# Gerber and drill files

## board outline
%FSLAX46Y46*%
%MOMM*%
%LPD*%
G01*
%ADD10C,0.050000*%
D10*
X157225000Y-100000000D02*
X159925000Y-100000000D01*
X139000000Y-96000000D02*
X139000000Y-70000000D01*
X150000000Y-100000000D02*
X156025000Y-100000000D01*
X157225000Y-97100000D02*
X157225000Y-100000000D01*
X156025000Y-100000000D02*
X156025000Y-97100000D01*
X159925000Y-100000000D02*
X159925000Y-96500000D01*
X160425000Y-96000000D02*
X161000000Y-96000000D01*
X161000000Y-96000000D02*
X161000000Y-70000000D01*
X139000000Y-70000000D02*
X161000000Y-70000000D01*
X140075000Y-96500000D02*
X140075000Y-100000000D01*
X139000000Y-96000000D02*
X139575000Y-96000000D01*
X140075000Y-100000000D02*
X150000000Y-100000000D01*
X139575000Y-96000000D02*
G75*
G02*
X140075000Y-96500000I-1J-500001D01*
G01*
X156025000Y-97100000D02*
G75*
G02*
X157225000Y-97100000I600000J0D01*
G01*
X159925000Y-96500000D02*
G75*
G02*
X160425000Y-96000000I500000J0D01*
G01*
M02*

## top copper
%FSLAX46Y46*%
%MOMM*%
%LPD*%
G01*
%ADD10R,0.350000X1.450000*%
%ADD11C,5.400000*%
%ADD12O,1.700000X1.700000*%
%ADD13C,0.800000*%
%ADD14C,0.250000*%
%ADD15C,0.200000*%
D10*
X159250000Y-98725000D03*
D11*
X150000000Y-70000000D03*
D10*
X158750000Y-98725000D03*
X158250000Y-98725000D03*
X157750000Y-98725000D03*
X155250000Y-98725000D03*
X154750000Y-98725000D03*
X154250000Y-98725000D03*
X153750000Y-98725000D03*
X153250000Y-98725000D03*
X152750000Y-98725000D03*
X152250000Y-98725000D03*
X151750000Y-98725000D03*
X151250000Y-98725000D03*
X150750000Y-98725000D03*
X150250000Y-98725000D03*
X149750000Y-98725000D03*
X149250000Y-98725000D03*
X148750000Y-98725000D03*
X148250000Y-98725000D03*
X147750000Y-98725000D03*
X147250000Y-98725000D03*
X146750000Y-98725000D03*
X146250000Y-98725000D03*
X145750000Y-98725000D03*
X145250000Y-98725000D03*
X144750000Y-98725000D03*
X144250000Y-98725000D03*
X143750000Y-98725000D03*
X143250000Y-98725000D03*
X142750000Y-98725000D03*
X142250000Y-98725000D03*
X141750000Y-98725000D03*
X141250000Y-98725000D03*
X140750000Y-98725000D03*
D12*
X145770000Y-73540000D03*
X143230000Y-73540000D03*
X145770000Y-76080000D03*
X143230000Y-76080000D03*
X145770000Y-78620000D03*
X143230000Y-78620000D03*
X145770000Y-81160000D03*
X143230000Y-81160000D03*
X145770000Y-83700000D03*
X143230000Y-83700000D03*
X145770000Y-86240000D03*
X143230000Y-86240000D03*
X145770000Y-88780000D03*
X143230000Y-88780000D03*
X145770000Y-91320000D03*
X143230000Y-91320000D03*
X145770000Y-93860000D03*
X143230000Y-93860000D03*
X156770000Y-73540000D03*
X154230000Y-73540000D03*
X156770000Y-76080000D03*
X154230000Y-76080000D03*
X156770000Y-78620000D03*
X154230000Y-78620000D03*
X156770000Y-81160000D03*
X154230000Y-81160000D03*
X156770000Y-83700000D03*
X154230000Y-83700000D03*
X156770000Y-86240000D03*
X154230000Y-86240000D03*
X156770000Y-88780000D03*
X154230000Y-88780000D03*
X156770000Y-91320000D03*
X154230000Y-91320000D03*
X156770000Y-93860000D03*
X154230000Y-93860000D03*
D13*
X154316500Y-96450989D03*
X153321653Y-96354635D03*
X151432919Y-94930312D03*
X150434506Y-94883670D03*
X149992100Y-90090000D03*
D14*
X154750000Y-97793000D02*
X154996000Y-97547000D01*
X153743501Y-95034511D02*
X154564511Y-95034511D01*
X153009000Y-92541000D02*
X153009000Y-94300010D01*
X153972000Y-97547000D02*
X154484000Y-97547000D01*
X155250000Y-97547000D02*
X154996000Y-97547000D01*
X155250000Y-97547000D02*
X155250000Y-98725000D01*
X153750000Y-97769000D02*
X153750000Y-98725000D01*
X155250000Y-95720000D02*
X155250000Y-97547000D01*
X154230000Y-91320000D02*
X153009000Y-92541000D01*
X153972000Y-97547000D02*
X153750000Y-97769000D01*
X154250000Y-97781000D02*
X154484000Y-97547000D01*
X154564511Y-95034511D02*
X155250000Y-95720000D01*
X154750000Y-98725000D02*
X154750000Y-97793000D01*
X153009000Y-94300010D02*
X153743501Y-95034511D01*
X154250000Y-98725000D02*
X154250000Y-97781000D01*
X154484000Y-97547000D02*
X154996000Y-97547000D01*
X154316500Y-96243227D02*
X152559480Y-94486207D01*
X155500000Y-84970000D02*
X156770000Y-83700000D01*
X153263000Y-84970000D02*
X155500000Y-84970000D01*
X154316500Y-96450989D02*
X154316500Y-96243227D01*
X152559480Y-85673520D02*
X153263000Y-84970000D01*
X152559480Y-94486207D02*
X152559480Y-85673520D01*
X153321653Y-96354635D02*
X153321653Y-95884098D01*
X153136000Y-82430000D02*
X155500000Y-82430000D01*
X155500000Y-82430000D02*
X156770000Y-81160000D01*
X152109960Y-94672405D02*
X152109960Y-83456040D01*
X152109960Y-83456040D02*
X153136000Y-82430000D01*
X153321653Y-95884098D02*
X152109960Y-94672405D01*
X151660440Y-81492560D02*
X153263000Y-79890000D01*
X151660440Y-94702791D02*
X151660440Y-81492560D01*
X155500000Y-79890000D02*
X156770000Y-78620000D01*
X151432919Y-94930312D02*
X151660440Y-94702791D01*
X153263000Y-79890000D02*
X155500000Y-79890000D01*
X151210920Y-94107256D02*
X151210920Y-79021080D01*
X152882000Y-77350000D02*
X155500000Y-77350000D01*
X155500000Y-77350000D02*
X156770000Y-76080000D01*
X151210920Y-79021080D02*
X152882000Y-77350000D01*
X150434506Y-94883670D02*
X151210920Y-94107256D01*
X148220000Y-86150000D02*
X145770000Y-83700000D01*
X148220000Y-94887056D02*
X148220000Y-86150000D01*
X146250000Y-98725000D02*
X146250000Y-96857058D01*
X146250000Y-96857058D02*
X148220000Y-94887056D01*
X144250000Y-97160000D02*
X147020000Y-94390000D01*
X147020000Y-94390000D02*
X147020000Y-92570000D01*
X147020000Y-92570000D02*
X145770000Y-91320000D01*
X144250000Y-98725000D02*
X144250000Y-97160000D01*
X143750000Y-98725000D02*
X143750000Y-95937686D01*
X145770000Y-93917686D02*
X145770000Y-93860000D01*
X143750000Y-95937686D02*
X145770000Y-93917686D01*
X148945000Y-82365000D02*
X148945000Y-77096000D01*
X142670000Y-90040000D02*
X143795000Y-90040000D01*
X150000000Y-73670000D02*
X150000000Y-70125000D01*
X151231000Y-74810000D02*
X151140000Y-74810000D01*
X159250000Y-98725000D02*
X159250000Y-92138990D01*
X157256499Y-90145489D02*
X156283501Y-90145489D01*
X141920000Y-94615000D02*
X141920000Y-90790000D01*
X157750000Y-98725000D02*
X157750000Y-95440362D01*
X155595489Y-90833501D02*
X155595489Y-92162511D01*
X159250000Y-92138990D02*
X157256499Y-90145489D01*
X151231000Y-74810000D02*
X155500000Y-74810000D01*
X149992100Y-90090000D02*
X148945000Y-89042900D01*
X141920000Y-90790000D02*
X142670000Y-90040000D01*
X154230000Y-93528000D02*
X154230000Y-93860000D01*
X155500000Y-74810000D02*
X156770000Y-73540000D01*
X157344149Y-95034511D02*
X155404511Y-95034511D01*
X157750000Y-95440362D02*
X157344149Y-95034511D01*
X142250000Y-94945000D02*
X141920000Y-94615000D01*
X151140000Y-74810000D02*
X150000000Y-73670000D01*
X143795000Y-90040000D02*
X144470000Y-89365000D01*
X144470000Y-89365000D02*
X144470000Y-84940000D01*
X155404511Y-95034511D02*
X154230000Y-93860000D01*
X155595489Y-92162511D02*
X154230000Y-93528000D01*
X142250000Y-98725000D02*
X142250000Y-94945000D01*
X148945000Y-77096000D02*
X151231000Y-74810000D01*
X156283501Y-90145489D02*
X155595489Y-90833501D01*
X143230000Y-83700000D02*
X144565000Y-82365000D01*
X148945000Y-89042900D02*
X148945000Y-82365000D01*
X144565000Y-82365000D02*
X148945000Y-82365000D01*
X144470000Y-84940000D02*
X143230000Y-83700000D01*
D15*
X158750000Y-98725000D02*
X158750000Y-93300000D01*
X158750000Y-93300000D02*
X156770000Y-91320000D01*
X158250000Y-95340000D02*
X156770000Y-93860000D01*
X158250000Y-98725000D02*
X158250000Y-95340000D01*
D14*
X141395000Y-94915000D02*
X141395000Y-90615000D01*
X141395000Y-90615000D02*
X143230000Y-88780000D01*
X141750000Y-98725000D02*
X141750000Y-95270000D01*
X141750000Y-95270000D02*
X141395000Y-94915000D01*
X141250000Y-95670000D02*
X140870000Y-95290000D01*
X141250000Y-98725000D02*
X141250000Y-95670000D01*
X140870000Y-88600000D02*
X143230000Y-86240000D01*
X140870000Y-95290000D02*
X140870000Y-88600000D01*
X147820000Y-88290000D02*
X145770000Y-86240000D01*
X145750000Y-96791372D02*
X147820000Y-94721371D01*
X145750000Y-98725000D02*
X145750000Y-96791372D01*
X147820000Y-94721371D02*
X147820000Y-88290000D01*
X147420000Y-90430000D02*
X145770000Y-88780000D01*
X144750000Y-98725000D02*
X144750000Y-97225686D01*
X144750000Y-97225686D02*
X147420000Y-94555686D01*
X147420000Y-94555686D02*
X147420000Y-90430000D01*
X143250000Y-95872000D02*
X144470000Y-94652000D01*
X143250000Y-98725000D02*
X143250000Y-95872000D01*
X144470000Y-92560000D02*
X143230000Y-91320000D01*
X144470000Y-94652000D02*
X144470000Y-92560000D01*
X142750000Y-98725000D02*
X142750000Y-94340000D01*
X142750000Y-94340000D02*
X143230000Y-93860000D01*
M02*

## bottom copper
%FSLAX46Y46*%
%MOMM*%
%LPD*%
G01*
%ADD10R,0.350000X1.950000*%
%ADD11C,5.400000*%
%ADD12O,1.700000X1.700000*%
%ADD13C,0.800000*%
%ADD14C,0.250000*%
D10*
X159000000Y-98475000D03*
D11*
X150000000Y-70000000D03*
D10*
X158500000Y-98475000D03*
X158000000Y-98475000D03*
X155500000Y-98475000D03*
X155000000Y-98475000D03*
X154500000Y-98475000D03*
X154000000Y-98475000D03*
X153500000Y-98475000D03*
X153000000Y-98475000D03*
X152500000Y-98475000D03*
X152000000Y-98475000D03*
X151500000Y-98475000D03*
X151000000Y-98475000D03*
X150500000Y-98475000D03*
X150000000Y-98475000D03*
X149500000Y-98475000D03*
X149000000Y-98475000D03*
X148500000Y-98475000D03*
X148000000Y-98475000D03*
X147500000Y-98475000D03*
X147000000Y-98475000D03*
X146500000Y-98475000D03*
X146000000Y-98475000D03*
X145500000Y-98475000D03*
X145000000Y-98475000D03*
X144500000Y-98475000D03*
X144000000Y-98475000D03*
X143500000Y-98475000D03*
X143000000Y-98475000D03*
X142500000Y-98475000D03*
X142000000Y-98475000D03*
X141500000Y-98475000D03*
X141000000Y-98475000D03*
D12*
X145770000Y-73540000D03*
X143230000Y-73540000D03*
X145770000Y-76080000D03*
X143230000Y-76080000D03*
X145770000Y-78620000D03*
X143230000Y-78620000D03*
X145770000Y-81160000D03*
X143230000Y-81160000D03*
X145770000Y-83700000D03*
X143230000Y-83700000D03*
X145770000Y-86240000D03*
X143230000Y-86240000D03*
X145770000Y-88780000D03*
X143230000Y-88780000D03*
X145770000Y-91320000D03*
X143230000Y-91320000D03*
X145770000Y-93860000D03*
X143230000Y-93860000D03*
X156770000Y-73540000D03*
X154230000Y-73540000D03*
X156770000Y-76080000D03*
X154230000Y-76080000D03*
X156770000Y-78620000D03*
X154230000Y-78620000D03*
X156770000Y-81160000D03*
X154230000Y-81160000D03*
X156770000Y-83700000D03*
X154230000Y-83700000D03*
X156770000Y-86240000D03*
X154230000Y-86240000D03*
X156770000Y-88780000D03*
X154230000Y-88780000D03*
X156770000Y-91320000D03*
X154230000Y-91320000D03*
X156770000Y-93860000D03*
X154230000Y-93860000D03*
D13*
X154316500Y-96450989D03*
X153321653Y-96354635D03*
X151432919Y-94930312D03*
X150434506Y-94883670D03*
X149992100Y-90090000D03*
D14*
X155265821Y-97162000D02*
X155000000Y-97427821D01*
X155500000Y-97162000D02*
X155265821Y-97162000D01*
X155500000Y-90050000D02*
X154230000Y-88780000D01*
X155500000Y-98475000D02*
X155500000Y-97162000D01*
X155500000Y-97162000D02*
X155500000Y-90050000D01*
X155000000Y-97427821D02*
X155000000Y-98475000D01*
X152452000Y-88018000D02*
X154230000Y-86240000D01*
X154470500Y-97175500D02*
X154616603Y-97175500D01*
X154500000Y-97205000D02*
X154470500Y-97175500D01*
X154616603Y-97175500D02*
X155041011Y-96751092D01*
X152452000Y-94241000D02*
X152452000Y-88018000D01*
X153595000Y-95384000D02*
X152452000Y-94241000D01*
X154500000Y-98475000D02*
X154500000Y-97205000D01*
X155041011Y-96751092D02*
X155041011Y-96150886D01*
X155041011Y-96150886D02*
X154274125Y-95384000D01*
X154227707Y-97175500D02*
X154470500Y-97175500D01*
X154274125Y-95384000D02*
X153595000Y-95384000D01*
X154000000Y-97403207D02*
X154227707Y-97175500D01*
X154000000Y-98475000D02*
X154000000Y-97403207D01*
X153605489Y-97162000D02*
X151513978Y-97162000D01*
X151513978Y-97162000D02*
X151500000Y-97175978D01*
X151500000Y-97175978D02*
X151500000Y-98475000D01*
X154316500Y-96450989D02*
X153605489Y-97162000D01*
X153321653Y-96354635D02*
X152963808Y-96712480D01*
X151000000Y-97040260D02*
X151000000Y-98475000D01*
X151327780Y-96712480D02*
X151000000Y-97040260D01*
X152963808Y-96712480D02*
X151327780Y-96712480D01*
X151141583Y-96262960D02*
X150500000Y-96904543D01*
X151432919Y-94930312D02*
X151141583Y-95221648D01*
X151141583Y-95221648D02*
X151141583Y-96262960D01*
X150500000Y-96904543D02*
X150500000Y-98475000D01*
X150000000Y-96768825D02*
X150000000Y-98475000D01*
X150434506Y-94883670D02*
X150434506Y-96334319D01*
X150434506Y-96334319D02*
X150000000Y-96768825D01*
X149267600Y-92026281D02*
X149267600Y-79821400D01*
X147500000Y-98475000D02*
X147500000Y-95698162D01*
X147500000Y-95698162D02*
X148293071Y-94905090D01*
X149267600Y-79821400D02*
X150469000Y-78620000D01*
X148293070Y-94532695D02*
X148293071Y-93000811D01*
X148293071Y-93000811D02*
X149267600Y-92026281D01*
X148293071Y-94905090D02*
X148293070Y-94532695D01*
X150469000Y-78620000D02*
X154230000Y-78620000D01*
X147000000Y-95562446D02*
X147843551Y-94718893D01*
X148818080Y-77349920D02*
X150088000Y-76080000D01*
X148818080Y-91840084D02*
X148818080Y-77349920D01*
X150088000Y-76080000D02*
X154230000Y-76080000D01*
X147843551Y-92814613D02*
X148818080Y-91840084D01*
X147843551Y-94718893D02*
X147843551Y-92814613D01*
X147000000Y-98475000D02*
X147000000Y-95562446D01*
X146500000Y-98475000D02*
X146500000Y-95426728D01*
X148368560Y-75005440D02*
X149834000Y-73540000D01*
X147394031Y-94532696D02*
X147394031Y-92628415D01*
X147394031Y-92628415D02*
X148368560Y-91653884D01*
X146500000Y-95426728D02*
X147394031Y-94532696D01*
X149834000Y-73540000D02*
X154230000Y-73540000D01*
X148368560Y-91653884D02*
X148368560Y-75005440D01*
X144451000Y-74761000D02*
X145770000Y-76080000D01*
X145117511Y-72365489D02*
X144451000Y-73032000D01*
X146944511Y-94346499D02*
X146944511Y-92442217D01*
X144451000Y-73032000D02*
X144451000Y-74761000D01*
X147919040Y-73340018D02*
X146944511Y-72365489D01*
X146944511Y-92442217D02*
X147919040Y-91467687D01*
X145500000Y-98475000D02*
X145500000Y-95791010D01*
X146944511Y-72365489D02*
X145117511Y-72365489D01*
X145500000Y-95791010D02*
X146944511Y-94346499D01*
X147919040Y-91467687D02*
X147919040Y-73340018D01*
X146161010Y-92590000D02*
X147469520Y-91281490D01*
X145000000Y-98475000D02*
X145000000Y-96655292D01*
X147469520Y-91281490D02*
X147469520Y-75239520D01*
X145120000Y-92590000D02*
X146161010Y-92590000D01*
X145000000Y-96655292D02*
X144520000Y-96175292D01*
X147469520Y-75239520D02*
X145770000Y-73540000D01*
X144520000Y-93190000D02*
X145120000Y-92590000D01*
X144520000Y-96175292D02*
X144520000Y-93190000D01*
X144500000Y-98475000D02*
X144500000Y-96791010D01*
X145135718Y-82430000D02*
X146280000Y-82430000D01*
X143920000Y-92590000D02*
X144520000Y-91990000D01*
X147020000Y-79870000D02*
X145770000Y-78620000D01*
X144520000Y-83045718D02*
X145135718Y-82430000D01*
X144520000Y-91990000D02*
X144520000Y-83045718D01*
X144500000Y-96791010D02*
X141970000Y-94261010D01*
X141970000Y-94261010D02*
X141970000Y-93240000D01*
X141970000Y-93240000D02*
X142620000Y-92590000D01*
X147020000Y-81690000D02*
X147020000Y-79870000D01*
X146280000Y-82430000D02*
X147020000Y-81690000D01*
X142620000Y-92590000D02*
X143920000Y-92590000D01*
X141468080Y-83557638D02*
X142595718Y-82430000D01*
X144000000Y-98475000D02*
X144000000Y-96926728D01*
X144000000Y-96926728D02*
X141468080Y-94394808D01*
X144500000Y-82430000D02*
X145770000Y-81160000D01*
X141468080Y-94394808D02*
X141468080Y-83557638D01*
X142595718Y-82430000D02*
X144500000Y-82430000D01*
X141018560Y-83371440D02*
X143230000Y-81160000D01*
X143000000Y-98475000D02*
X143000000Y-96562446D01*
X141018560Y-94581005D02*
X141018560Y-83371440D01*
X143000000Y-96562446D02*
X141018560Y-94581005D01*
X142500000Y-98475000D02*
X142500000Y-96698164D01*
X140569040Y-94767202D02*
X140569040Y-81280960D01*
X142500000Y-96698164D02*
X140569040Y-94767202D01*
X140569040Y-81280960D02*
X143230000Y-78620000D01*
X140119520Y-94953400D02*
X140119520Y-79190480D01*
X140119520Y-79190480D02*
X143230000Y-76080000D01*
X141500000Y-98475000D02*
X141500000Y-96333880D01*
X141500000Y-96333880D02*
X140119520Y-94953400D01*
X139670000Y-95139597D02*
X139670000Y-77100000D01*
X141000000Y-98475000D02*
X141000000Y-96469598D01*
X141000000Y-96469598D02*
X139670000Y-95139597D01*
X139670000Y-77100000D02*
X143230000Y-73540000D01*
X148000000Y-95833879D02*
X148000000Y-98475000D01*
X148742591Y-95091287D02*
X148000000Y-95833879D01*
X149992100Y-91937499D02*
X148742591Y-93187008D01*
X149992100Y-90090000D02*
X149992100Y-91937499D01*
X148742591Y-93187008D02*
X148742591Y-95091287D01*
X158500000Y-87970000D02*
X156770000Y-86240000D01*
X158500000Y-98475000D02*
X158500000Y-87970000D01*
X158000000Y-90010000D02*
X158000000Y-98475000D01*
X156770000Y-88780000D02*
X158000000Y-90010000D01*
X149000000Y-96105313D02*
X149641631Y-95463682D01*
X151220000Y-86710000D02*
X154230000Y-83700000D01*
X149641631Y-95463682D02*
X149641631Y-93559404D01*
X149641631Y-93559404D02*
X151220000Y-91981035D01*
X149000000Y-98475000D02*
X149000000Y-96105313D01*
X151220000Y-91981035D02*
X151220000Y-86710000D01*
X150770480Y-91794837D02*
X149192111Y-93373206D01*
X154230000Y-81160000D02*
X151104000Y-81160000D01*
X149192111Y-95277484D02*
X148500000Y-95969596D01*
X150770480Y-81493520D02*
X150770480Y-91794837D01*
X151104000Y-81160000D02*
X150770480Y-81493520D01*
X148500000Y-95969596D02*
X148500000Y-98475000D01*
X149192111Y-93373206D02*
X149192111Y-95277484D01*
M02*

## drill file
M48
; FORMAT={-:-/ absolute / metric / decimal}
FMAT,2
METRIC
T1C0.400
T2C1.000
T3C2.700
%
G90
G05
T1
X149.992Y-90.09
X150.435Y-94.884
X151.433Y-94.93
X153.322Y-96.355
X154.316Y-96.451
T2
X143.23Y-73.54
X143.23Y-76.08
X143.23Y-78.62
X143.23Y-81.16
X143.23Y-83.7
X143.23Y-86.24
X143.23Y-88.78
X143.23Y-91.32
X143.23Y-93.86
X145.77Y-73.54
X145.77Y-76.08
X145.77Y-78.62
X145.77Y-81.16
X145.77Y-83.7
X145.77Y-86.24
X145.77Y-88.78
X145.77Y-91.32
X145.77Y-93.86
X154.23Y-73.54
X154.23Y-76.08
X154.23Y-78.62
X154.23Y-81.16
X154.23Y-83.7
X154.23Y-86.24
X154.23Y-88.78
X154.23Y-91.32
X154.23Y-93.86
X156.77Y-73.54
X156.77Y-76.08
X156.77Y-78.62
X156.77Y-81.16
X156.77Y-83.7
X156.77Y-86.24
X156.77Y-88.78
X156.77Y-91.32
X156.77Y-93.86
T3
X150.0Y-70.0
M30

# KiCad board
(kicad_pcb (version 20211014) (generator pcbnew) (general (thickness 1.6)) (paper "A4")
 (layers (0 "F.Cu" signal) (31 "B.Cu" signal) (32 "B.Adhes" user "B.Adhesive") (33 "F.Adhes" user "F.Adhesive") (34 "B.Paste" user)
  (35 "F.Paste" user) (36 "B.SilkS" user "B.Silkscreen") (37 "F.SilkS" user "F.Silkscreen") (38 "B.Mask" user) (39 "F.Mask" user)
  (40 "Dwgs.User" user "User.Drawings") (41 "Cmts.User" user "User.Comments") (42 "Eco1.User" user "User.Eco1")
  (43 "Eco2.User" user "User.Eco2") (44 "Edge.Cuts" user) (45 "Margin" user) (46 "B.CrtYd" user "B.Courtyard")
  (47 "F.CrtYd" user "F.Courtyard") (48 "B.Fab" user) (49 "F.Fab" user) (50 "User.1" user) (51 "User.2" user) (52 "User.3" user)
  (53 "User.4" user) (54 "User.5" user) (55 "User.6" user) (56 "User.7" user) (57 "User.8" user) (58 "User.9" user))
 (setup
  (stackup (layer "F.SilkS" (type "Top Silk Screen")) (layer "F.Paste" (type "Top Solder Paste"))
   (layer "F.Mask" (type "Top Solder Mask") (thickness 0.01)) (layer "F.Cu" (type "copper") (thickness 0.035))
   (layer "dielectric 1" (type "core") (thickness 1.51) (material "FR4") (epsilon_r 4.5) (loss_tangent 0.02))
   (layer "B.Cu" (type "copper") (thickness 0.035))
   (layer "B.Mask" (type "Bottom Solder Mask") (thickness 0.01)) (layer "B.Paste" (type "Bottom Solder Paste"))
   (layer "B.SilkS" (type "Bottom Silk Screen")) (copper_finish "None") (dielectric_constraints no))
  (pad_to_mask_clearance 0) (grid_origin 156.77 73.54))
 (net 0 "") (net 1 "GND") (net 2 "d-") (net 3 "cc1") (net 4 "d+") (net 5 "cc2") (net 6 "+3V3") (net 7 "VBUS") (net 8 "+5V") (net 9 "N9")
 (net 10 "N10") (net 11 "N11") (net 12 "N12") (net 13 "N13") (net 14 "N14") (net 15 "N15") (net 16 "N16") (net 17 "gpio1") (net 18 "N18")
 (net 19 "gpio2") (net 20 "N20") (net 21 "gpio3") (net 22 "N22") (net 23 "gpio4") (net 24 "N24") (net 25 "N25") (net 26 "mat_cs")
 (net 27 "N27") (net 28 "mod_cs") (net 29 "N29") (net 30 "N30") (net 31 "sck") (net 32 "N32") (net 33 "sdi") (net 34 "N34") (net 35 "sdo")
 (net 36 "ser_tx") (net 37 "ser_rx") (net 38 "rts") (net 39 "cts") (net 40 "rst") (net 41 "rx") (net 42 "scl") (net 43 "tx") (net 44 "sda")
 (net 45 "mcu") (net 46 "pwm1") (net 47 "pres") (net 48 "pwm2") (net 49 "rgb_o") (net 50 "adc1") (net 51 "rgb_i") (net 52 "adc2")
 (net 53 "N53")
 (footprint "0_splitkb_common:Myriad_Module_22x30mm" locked (layer "F.Cu") (at 150 100)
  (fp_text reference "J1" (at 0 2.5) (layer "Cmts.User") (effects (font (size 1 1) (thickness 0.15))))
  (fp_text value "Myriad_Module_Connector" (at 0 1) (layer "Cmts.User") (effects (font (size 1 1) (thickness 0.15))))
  (fp_line (start 7.225 0) (end 9.925 0) (layer "Edge.Cuts") (width 0.05))
  (fp_line (start -11 -4) (end -11 -30) (layer "Edge.Cuts") (width 0.05))
  (fp_line (start 0 0) (end 6.025 0) (layer "Edge.Cuts") (width 0.05))
  (fp_line (start 7.225 -2.9) (end 7.225 0) (layer "Edge.Cuts") (width 0.05))
  (fp_line (start 6.025 0) (end 6.025 -2.9) (layer "Edge.Cuts") (width 0.05))
  (fp_line (start 9.925 0) (end 9.925 -3.5) (layer "Edge.Cuts") (width 0.05))
  (fp_line (start 10.425 -4) (end 11 -4) (layer "Edge.Cuts") (width 0.05))
  (fp_line (start 11 -4) (end 11 -30) (layer "Edge.Cuts") (width 0.05))
  (fp_line (start -11 -30) (end 11 -30) (layer "Edge.Cuts") (width 0.05))
  (fp_line (start -9.925 -3.5) (end -9.925 0) (layer "Edge.Cuts") (width 0.05))
  (fp_line (start -11 -4) (end -10.425 -4) (layer "Edge.Cuts") (width 0.05))
  (fp_line (start -9.925 0) (end 0 0) (layer "Edge.Cuts") (width 0.05))
  (fp_arc (start -10.425 -4) (mid -10.071447 -3.853553) (end -9.925 -3.5) (layer "Edge.Cuts") (width 0.05))
  (fp_arc (start 6.025 -2.9) (mid 6.625 -3.5) (end 7.225 -2.9) (layer "Edge.Cuts") (width 0.05))
  (fp_arc (start 9.925 -3.5) (mid 10.071447 -3.853553) (end 10.425 -4) (layer "Edge.Cuts") (width 0.05))
  (pad "1" smd rect locked (at 9.25 -1.275) (size 0.35 1.45) (layers "F.Cu") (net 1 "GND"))
  (pad "2" smd rect locked (at 9 -1.525) (size 0.35 1.95) (layers "B.Cu") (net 1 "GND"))
  (pad "2" thru_hole circle locked (at 0 -30) (size 5.4 5.4) (drill 2.7) (layers *.Cu *.Mask) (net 1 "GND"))
  (pad "3" smd rect locked (at 8.75 -1.275) (size 0.35 1.45) (layers "F.Cu") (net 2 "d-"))
  (pad "4" smd rect locked (at 8.5 -1.525) (size 0.35 1.95) (layers "B.Cu") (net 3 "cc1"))
  (pad "5" smd rect locked (at 8.25 -1.275) (size 0.35 1.45) (layers "F.Cu") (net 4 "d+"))
  (pad "6" smd rect locked (at 8 -1.525) (size 0.35 1.95) (layers "B.Cu") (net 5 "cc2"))
  (pad "7" smd rect locked (at 7.75 -1.275) (size 0.35 1.45) (layers "F.Cu") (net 1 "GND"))
  (pad "16" smd rect locked (at 5.5 -1.525) (size 0.35 1.95) (layers "B.Cu") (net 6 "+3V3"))
  (pad "17" smd rect locked (at 5.25 -1.275) (size 0.35 1.45) (layers "F.Cu") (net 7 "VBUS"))
  (pad "18" smd rect locked (at 5 -1.525) (size 0.35 1.95) (layers "B.Cu") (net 6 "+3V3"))
  (pad "19" smd rect locked (at 4.75 -1.275) (size 0.35 1.45) (layers "F.Cu") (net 7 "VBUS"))
  (pad "20" smd rect locked (at 4.5 -1.525) (size 0.35 1.95) (layers "B.Cu") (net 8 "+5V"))
  (pad "21" smd rect locked (at 4.25 -1.275) (size 0.35 1.45) (layers "F.Cu") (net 7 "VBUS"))
  (pad "22" smd rect locked (at 4 -1.525) (size 0.35 1.95) (layers "B.Cu") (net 8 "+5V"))
  (pad "23" smd rect locked (at 3.75 -1.275) (size 0.35 1.45) (layers "F.Cu") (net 7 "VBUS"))
  (pad "24" smd rect locked (at 3.5 -1.525) (size 0.35 1.95) (layers "B.Cu") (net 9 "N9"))
  (pad "25" smd rect locked (at 3.25 -1.275) (size 0.35 1.45) (layers "F.Cu") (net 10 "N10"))
  (pad "26" smd rect locked (at 3 -1.525) (size 0.35 1.95) (layers "B.Cu") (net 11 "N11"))
  (pad "27" smd rect locked (at 2.75 -1.275) (size 0.35 1.45) (layers "F.Cu") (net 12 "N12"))
  (pad "28" smd rect locked (at 2.5 -1.525) (size 0.35 1.95) (layers "B.Cu") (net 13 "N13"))
  (pad "29" smd rect locked (at 2.25 -1.275) (size 0.35 1.45) (layers "F.Cu") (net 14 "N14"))
  (pad "30" smd rect locked (at 2 -1.525) (size 0.35 1.95) (layers "B.Cu") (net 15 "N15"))
  (pad "31" smd rect locked (at 1.75 -1.275) (size 0.35 1.45) (layers "F.Cu") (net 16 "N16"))
  (pad "32" smd rect locked (at 1.5 -1.525) (size 0.35 1.95) (layers "B.Cu") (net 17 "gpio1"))
  (pad "33" smd rect locked (at 1.25 -1.275) (size 0.35 1.45) (layers "F.Cu") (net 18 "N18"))
  (pad "34" smd rect locked (at 1 -1.525) (size 0.35 1.95) (layers "B.Cu") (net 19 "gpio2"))
  (pad "35" smd rect locked (at 0.75 -1.275) (size 0.35 1.45) (layers "F.Cu") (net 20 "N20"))
  (pad "36" smd rect locked (at 0.5 -1.525) (size 0.35 1.95) (layers "B.Cu") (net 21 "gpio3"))
  (pad "37" smd rect locked (at 0.25 -1.275) (size 0.35 1.45) (layers "F.Cu") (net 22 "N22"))
  (pad "38" smd rect locked (at 0 -1.525) (size 0.35 1.95) (layers "B.Cu") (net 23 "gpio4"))
  (pad "39" smd rect locked (at -0.25 -1.275) (size 0.35 1.45) (layers "F.Cu") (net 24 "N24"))
  (pad "40" smd rect locked (at -0.5 -1.525) (size 0.35 1.95) (layers "B.Cu") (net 1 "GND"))
  (pad "41" smd rect locked (at -0.75 -1.275) (size 0.35 1.45) (layers "F.Cu") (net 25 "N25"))
  (pad "42" smd rect locked (at -1 -1.525) (size 0.35 1.95) (layers "B.Cu") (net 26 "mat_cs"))
  (pad "43" smd rect locked (at -1.25 -1.275) (size 0.35 1.45) (layers "F.Cu") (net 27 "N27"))
  (pad "44" smd rect locked (at -1.5 -1.525) (size 0.35 1.95) (layers "B.Cu") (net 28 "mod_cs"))
  (pad "45" smd rect locked (at -1.75 -1.275) (size 0.35 1.45) (layers "F.Cu") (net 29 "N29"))
  (pad "46" smd rect locked (at -2 -1.525) (size 0.35 1.95) (layers "B.Cu") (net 1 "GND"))
  (pad "47" smd rect locked (at -2.25 -1.275) (size 0.35 1.45) (layers "F.Cu") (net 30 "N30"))
  (pad "48" smd rect locked (at -2.5 -1.525) (size 0.35 1.95) (layers "B.Cu") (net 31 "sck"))
  (pad "49" smd rect locked (at -2.75 -1.275) (size 0.35 1.45) (layers "F.Cu") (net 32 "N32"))
  (pad "50" smd rect locked (at -3 -1.525) (size 0.35 1.95) (layers "B.Cu") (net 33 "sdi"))
  (pad "51" smd rect locked (at -3.25 -1.275) (size 0.35 1.45) (layers "F.Cu") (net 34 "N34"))
  (pad "52" smd rect locked (at -3.5 -1.525) (size 0.35 1.95) (layers "B.Cu") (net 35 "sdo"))
  (pad "53" smd rect locked (at -3.75 -1.275) (size 0.35 1.45) (layers "F.Cu") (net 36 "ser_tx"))
  (pad "54" smd rect locked (at -4 -1.525) (size 0.35 1.95) (layers "B.Cu") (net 1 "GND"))
  (pad "55" smd rect locked (at -4.25 -1.275) (size 0.35 1.45) (layers "F.Cu") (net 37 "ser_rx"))
  (pad "56" smd rect locked (at -4.5 -1.525) (size 0.35 1.95) (layers "B.Cu") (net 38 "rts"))
  (pad "57" smd rect locked (at -4.75 -1.275) (size 0.35 1.45) (layers "F.Cu") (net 1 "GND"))
  (pad "58" smd rect locked (at -5 -1.525) (size 0.35 1.95) (layers "B.Cu") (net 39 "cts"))
  (pad "59" smd rect locked (at -5.25 -1.275) (size 0.35 1.45) (layers "F.Cu") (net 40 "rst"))
  (pad "60" smd rect locked (at -5.5 -1.525) (size 0.35 1.95) (layers "B.Cu") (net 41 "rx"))
  (pad "61" smd rect locked (at -5.75 -1.275) (size 0.35 1.45) (layers "F.Cu") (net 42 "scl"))
  (pad "62" smd rect locked (at -6 -1.525) (size 0.35 1.95) (layers "B.Cu") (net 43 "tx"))
  (pad "63" smd rect locked (at -6.25 -1.275) (size 0.35 1.45) (layers "F.Cu") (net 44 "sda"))
  (pad "64" smd rect locked (at -6.5 -1.525) (size 0.35 1.95) (layers "B.Cu") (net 1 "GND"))
  (pad "65" smd rect locked (at -6.75 -1.275) (size 0.35 1.45) (layers "F.Cu") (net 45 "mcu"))
  (pad "66" smd rect locked (at -7 -1.525) (size 0.35 1.95) (layers "B.Cu") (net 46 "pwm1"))
  (pad "67" smd rect locked (at -7.25 -1.275) (size 0.35 1.45) (layers "F.Cu") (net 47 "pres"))
  (pad "68" smd rect locked (at -7.5 -1.525) (size 0.35 1.95) (layers "B.Cu") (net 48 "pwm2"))
  (pad "69" smd rect locked (at -7.75 -1.275) (size 0.35 1.45) (layers "F.Cu") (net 1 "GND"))
  (pad "70" smd rect locked (at -8 -1.525) (size 0.35 1.95) (layers "B.Cu") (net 1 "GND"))
  (pad "71" smd rect locked (at -8.25 -1.275) (size 0.35 1.45) (layers "F.Cu") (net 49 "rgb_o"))
  (pad "72" smd rect locked (at -8.5 -1.525) (size 0.35 1.95) (layers "B.Cu") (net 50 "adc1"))
  (pad "73" smd rect locked (at -8.75 -1.275) (size 0.35 1.45) (layers "F.Cu") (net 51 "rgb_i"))
  (pad "74" smd rect locked (at -9 -1.525) (size 0.35 1.95) (layers "B.Cu") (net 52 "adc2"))
  (pad "75" smd rect locked (at -9.25 -1.275) (size 0.35 1.45) (layers "F.Cu") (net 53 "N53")))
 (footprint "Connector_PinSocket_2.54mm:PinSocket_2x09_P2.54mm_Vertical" (layer "F.Cu") (at 145.77 73.54)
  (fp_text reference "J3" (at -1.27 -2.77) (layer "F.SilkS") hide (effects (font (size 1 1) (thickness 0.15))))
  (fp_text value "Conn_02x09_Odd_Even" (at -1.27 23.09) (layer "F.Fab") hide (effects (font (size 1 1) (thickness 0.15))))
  (pad "1" thru_hole oval (at 0 0) (size 1.7 1.7) (drill 1) (layers *.Cu *.Mask) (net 39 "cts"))
  (pad "2" thru_hole oval (at -2.54 0) (size 1.7 1.7) (drill 1) (layers *.Cu *.Mask) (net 52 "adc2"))
  (pad "3" thru_hole oval (at 0 2.54) (size 1.7 1.7) (drill 1) (layers *.Cu *.Mask) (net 38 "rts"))
  (pad "4" thru_hole oval (at -2.54 2.54) (size 1.7 1.7) (drill 1) (layers *.Cu *.Mask) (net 50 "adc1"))
  (pad "5" thru_hole oval (at 0 5.08) (size 1.7 1.7) (drill 1) (layers *.Cu *.Mask) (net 41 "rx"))
  (pad "6" thru_hole oval (at -2.54 5.08) (size 1.7 1.7) (drill 1) (layers *.Cu *.Mask) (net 48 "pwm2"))
  (pad "7" thru_hole oval (at 0 7.62) (size 1.7 1.7) (drill 1) (layers *.Cu *.Mask) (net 43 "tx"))
  (pad "8" thru_hole oval (at -2.54 7.62) (size 1.7 1.7) (drill 1) (layers *.Cu *.Mask) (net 46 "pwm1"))
  (pad "9" thru_hole oval (at 0 10.16) (size 1.7 1.7) (drill 1) (layers *.Cu *.Mask) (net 36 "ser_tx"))
  (pad "10" thru_hole oval (at -2.54 10.16) (size 1.7 1.7) (drill 1) (layers *.Cu *.Mask) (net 1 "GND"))
  (pad "11" thru_hole oval (at 0 12.7) (size 1.7 1.7) (drill 1) (layers *.Cu *.Mask) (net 37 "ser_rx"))
  (pad "12" thru_hole oval (at -2.54 12.7) (size 1.7 1.7) (drill 1) (layers *.Cu *.Mask) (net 51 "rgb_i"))
  (pad "13" thru_hole oval (at 0 15.24) (size 1.7 1.7) (drill 1) (layers *.Cu *.Mask) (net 40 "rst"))
  (pad "14" thru_hole oval (at -2.54 15.24) (size 1.7 1.7) (drill 1) (layers *.Cu *.Mask) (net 49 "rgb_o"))
  (pad "15" thru_hole oval (at 0 17.78) (size 1.7 1.7) (drill 1) (layers *.Cu *.Mask) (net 42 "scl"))
  (pad "16" thru_hole oval (at -2.54 17.78) (size 1.7 1.7) (drill 1) (layers *.Cu *.Mask) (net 45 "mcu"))
  (pad "17" thru_hole oval (at 0 20.32) (size 1.7 1.7) (drill 1) (layers *.Cu *.Mask) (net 44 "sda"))
  (pad "18" thru_hole oval (at -2.54 20.32) (size 1.7 1.7) (drill 1) (layers *.Cu *.Mask) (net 47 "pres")))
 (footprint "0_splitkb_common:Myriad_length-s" (layer "F.Cu") (at 148.8 96.5)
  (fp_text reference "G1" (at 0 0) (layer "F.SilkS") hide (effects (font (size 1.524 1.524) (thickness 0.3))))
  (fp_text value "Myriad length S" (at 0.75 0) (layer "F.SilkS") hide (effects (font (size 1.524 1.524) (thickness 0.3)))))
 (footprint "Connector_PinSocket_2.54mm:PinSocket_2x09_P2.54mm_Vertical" (layer "F.Cu") (at 156.77 73.54)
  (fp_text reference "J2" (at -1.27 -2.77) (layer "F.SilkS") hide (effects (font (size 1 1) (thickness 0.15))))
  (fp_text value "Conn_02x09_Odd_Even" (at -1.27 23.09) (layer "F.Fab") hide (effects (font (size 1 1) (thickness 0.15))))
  (pad "1" thru_hole oval (at 0 0) (size 1.7 1.7) (drill 1) (layers *.Cu *.Mask) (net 1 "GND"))
  (pad "2" thru_hole oval (at -2.54 0) (size 1.7 1.7) (drill 1) (layers *.Cu *.Mask) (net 35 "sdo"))
  (pad "3" thru_hole oval (at 0 2.54) (size 1.7 1.7) (drill 1) (layers *.Cu *.Mask) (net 23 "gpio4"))
  (pad "4" thru_hole oval (at -2.54 2.54) (size 1.7 1.7) (drill 1) (layers *.Cu *.Mask) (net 33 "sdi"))
  (pad "5" thru_hole oval (at 0 5.08) (size 1.7 1.7) (drill 1) (layers *.Cu *.Mask) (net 21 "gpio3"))
  (pad "6" thru_hole oval (at -2.54 5.08) (size 1.7 1.7) (drill 1) (layers *.Cu *.Mask) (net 31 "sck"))
  (pad "7" thru_hole oval (at 0 7.62) (size 1.7 1.7) (drill 1) (layers *.Cu *.Mask) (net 19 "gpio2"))
  (pad "8" thru_hole oval (at -2.54 7.62) (size 1.7 1.7) (drill 1) (layers *.Cu *.Mask) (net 28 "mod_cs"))
  (pad "9" thru_hole oval (at 0 10.16) (size 1.7 1.7) (drill 1) (layers *.Cu *.Mask) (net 17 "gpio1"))
  (pad "10" thru_hole oval (at -2.54 10.16) (size 1.7 1.7) (drill 1) (layers *.Cu *.Mask) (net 26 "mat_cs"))
  (pad "11" thru_hole oval (at 0 12.7) (size 1.7 1.7) (drill 1) (layers *.Cu *.Mask) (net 3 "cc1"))
  (pad "12" thru_hole oval (at -2.54 12.7) (size 1.7 1.7) (drill 1) (layers *.Cu *.Mask) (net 8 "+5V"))
  (pad "13" thru_hole oval (at 0 15.24) (size 1.7 1.7) (drill 1) (layers *.Cu *.Mask) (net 5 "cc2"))
  (pad "14" thru_hole oval (at -2.54 15.24) (size 1.7 1.7) (drill 1) (layers *.Cu *.Mask) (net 6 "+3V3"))
  (pad "15" thru_hole oval (at 0 17.78) (size 1.7 1.7) (drill 1) (layers *.Cu *.Mask) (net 2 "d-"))
  (pad "16" thru_hole oval (at -2.54 17.78) (size 1.7 1.7) (drill 1) (layers *.Cu *.Mask) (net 7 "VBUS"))
  (pad "17" thru_hole oval (at 0 20.32) (size 1.7 1.7) (drill 1) (layers *.Cu *.Mask) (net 4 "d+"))
  (pad "18" thru_hole oval (at -2.54 20.32) (size 1.7 1.7) (drill 1) (layers *.Cu *.Mask) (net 1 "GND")))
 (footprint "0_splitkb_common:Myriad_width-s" (layer "F.Cu") (at 151.2 96.5)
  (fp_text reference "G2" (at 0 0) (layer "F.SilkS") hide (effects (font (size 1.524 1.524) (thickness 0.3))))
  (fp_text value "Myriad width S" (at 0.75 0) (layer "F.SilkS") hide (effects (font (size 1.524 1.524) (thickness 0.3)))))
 (segment (start 155.265821 97.162) (end 155 97.427821) (width 0.25) (layer "B.Cu") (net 6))
 (segment (start 155.5 97.162) (end 155.265821 97.162) (width 0.25) (layer "B.Cu") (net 6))
 (segment (start 155.5 90.05) (end 154.23 88.78) (width 0.25) (layer "B.Cu") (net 6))
 (segment (start 155.5 98.475) (end 155.5 97.162) (width 0.25) (layer "B.Cu") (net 6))
 (segment (start 155.5 97.162) (end 155.5 90.05) (width 0.25) (layer "B.Cu") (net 6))
 (segment (start 155 97.427821) (end 155 98.475) (width 0.25) (layer "B.Cu") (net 6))
 (segment (start 154.75 97.793) (end 154.996 97.547) (width 0.25) (layer "F.Cu") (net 7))
 (segment (start 153.743501 95.034511) (end 154.564511 95.034511) (width 0.25) (layer "F.Cu") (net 7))
 (segment (start 153.009 92.541) (end 153.009 94.30001) (width 0.25) (layer "F.Cu") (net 7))
 (segment (start 153.972 97.547) (end 154.484 97.547) (width 0.25) (layer "F.Cu") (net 7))
 (segment (start 155.25 97.547) (end 154.996 97.547) (width 0.25) (layer "F.Cu") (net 7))
 (segment (start 155.25 97.547) (end 155.25 98.725) (width 0.25) (layer "F.Cu") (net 7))
 (segment (start 153.75 97.769) (end 153.75 98.725) (width 0.25) (layer "F.Cu") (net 7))
 (segment (start 155.25 95.72) (end 155.25 97.547) (width 0.25) (layer "F.Cu") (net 7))
 (segment (start 154.23 91.32) (end 153.009 92.541) (width 0.25) (layer "F.Cu") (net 7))
 (segment (start 153.972 97.547) (end 153.75 97.769) (width 0.25) (layer "F.Cu") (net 7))
 (segment (start 154.25 97.781) (end 154.484 97.547) (width 0.25) (layer "F.Cu") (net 7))
 (segment (start 154.564511 95.034511) (end 155.25 95.72) (width 0.25) (layer "F.Cu") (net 7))
 (segment (start 154.75 98.725) (end 154.75 97.793) (width 0.25) (layer "F.Cu") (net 7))
 (segment (start 153.009 94.30001) (end 153.743501 95.034511) (width 0.25) (layer "F.Cu") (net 7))
 (segment (start 154.25 98.725) (end 154.25 97.781) (width 0.25) (layer "F.Cu") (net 7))
 (segment (start 154.484 97.547) (end 154.996 97.547) (width 0.25) (layer "F.Cu") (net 7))
 (segment (start 152.452 88.018) (end 154.23 86.24) (width 0.25) (layer "B.Cu") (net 8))
 (segment (start 154.4705 97.1755) (end 154.616603 97.1755) (width 0.25) (layer "B.Cu") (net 8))
 (segment (start 154.5 97.205) (end 154.4705 97.1755) (width 0.25) (layer "B.Cu") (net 8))
 (segment (start 154.616603 97.1755) (end 155.041011 96.751092) (width 0.25) (layer "B.Cu") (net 8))
 (segment (start 152.452 94.241) (end 152.452 88.018) (width 0.25) (layer "B.Cu") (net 8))
 (segment (start 153.595 95.384) (end 152.452 94.241) (width 0.25) (layer "B.Cu") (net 8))
 (segment (start 154.5 98.475) (end 154.5 97.205) (width 0.25) (layer "B.Cu") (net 8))
 (segment (start 155.041011 96.751092) (end 155.041011 96.150886) (width 0.25) (layer "B.Cu") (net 8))
 (segment (start 155.041011 96.150886) (end 154.274125 95.384) (width 0.25) (layer "B.Cu") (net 8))
 (segment (start 154.227707 97.1755) (end 154.4705 97.1755) (width 0.25) (layer "B.Cu") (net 8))
 (segment (start 154.274125 95.384) (end 153.595 95.384) (width 0.25) (layer "B.Cu") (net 8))
 (segment (start 154 97.403207) (end 154.227707 97.1755) (width 0.25) (layer "B.Cu") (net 8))
 (segment (start 154 98.475) (end 154 97.403207) (width 0.25) (layer "B.Cu") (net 8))
 (segment (start 154.3165 96.243227) (end 152.55948 94.486207) (width 0.25) (layer "F.Cu") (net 17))
 (segment (start 155.5 84.97) (end 156.77 83.7) (width 0.25) (layer "F.Cu") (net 17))
 (segment (start 153.263 84.97) (end 155.5 84.97) (width 0.25) (layer "F.Cu") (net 17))
 (segment (start 154.3165 96.450989) (end 154.3165 96.243227) (width 0.25) (layer "F.Cu") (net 17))
 (segment (start 152.55948 85.67352) (end 153.263 84.97) (width 0.25) (layer "F.Cu") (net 17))
 (segment (start 152.55948 94.486207) (end 152.55948 85.67352) (width 0.25) (layer "F.Cu") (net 17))
 (via (at 154.3165 96.450989) (size 0.8) (drill 0.4) (layers "F.Cu" "B.Cu") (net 17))
 (segment (start 153.605489 97.162) (end 151.513978 97.162) (width 0.25) (layer "B.Cu") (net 17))
 (segment (start 151.513978 97.162) (end 151.5 97.175978) (width 0.25) (layer "B.Cu") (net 17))
 (segment (start 151.5 97.175978) (end 151.5 98.475) (width 0.25) (layer "B.Cu") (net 17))
 (segment (start 154.3165 96.450989) (end 153.605489 97.162) (width 0.25) (layer "B.Cu") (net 17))
 (segment (start 153.321653 96.354635) (end 153.321653 95.884098) (width 0.25) (layer "F.Cu") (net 19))
 (segment (start 153.136 82.43) (end 155.5 82.43) (width 0.25) (layer "F.Cu") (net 19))
 (segment (start 155.5 82.43) (end 156.77 81.16) (width 0.25) (layer "F.Cu") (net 19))
 (segment (start 152.10996 94.672405) (end 152.10996 83.45604) (width 0.25) (layer "F.Cu") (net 19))
 (segment (start 152.10996 83.45604) (end 153.136 82.43) (width 0.25) (layer "F.Cu") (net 19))
 (segment (start 153.321653 95.884098) (end 152.10996 94.672405) (width 0.25) (layer "F.Cu") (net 19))
 (via (at 153.321653 96.354635) (size 0.8) (drill 0.4) (layers "F.Cu" "B.Cu") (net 19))
 (segment (start 153.321653 96.354635) (end 152.963808 96.71248) (width 0.25) (layer "B.Cu") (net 19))
 (segment (start 151 97.04026) (end 151 98.475) (width 0.25) (layer "B.Cu") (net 19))
 (segment (start 151.32778 96.71248) (end 151 97.04026) (width 0.25) (layer "B.Cu") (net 19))
 (segment (start 152.963808 96.71248) (end 151.32778 96.71248) (width 0.25) (layer "B.Cu") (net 19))
 (segment (start 151.66044 81.49256) (end 153.263 79.89) (width 0.25) (layer "F.Cu") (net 21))
 (segment (start 151.66044 94.702791) (end 151.66044 81.49256) (width 0.25) (layer "F.Cu") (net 21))
 (segment (start 155.5 79.89) (end 156.77 78.62) (width 0.25) (layer "F.Cu") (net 21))
 (segment (start 151.432919 94.930312) (end 151.66044 94.702791) (width 0.25) (layer "F.Cu") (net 21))
 (segment (start 153.263 79.89) (end 155.5 79.89) (width 0.25) (layer "F.Cu") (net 21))
 (via (at 151.432919 94.930312) (size 0.8) (drill 0.4) (layers "F.Cu" "B.Cu") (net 21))
 (segment (start 151.141583 96.26296) (end 150.5 96.904543) (width 0.25) (layer "B.Cu") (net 21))
 (segment (start 151.432919 94.930312) (end 151.141583 95.221648) (width 0.25) (layer "B.Cu") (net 21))
 (segment (start 151.141583 95.221648) (end 151.141583 96.26296) (width 0.25) (layer "B.Cu") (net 21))
 (segment (start 150.5 96.904543) (end 150.5 98.475) (width 0.25) (layer "B.Cu") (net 21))
 (segment (start 151.21092 94.107256) (end 151.21092 79.02108) (width 0.25) (layer "F.Cu") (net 23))
 (segment (start 152.882 77.35) (end 155.5 77.35) (width 0.25) (layer "F.Cu") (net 23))
 (segment (start 155.5 77.35) (end 156.77 76.08) (width 0.25) (layer "F.Cu") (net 23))
 (segment (start 151.21092 79.02108) (end 152.882 77.35) (width 0.25) (layer "F.Cu") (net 23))
 (segment (start 150.434506 94.88367) (end 151.21092 94.107256) (width 0.25) (layer "F.Cu") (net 23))
 (via (at 150.434506 94.88367) (size 0.8) (drill 0.4) (layers "F.Cu" "B.Cu") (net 23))
 (segment (start 150 96.768825) (end 150 98.475) (width 0.25) (layer "B.Cu") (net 23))
 (segment (start 150.434506 94.88367) (end 150.434506 96.334319) (width 0.25) (layer "B.Cu") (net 23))
 (segment (start 150.434506 96.334319) (end 150 96.768825) (width 0.25) (layer "B.Cu") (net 23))
 (segment (start 149.2676 92.026281) (end 149.2676 79.8214) (width 0.25) (layer "B.Cu") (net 31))
 (segment (start 147.5 98.475) (end 147.5 95.698162) (width 0.25) (layer "B.Cu") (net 31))
 (segment (start 147.5 95.698162) (end 148.293071 94.90509) (width 0.25) (layer "B.Cu") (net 31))
 (segment (start 149.2676 79.8214) (end 150.469 78.62) (width 0.25) (layer "B.Cu") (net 31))
 (segment (start 148.29307 94.532695) (end 148.293071 93.000811) (width 0.25) (layer "B.Cu") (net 31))
 (segment (start 148.293071 93.000811) (end 149.2676 92.026281) (width 0.25) (layer "B.Cu") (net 31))
 (segment (start 148.293071 94.90509) (end 148.29307 94.532695) (width 0.25) (layer "B.Cu") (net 31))
 (segment (start 150.469 78.62) (end 154.23 78.62) (width 0.25) (layer "B.Cu") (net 31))
 (segment (start 147 95.562446) (end 147.843551 94.718893) (width 0.25) (layer "B.Cu") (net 33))
 (segment (start 148.81808 77.34992) (end 150.088 76.08) (width 0.25) (layer "B.Cu") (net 33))
 (segment (start 148.81808 91.840084) (end 148.81808 77.34992) (width 0.25) (layer "B.Cu") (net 33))
 (segment (start 150.088 76.08) (end 154.23 76.08) (width 0.25) (layer "B.Cu") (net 33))
 (segment (start 147.843551 92.814613) (end 148.81808 91.840084) (width 0.25) (layer "B.Cu") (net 33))
 (segment (start 147.843551 94.718893) (end 147.843551 92.814613) (width 0.25) (layer "B.Cu") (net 33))
 (segment (start 147 98.475) (end 147 95.562446) (width 0.25) (layer "B.Cu") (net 33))
 (segment (start 146.5 98.475) (end 146.5 95.426728) (width 0.25) (layer "B.Cu") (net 35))
 (segment (start 148.36856 75.00544) (end 149.834 73.54) (width 0.25) (layer "B.Cu") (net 35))
 (segment (start 147.394031 94.532696) (end 147.394031 92.628415) (width 0.25) (layer "B.Cu") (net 35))
 (segment (start 147.394031 92.628415) (end 148.36856 91.653884) (width 0.25) (layer "B.Cu") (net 35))
 (segment (start 146.5 95.426728) (end 147.394031 94.532696) (width 0.25) (layer "B.Cu") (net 35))
 (segment (start 149.834 73.54) (end 154.23 73.54) (width 0.25) (layer "B.Cu") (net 35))
 (segment (start 148.36856 91.653884) (end 148.36856 75.00544) (width 0.25) (layer "B.Cu") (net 35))
 (segment (start 148.22 86.15) (end 145.77 83.7) (width 0.25) (layer "F.Cu") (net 36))
 (segment (start 148.22 94.887056) (end 148.22 86.15) (width 0.25) (layer "F.Cu") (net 36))
 (segment (start 146.25 98.725) (end 146.25 96.857058) (width 0.25) (layer "F.Cu") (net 36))
 (segment (start 146.25 96.857058) (end 148.22 94.887056) (width 0.25) (layer "F.Cu") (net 36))
 (segment (start 144.451 74.761) (end 145.77 76.08) (width 0.25) (layer "B.Cu") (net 38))
 (segment (start 145.117511 72.365489) (end 144.451 73.032) (width 0.25) (layer "B.Cu") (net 38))
 (segment (start 146.944511 94.346499) (end 146.944511 92.442217) (width 0.25) (layer "B.Cu") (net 38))
 (segment (start 144.451 73.032) (end 144.451 74.761) (width 0.25) (layer "B.Cu") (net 38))
 (segment (start 147.91904 73.340018) (end 146.944511 72.365489) (width 0.25) (layer "B.Cu") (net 38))
 (segment (start 146.944511 92.442217) (end 147.91904 91.467687) (width 0.25) (layer "B.Cu") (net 38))
 (segment (start 145.5 98.475) (end 145.5 95.79101) (width 0.25) (layer "B.Cu") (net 38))
 (segment (start 146.944511 72.365489) (end 145.117511 72.365489) (width 0.25) (layer "B.Cu") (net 38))
 (segment (start 145.5 95.79101) (end 146.944511 94.346499) (width 0.25) (layer "B.Cu") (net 38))
 (segment (start 147.91904 91.467687) (end 147.91904 73.340018) (width 0.25) (layer "B.Cu") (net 38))
 (segment (start 146.16101 92.59) (end 147.46952 91.28149) (width 0.25) (layer "B.Cu") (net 39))
 (segment (start 145 98.475) (end 145 96.655292) (width 0.25) (layer "B.Cu") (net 39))
 (segment (start 147.46952 91.28149) (end 147.46952 75.23952) (width 0.25) (layer "B.Cu") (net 39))
 (segment (start 145.12 92.59) (end 146.16101 92.59) (width 0.25) (layer "B.Cu") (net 39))
 (segment (start 145 96.655292) (end 144.52 96.175292) (width 0.25) (layer "B.Cu") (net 39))
 (segment (start 147.46952 75.23952) (end 145.77 73.54) (width 0.25) (layer "B.Cu") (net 39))
 (segment (start 144.52 93.19) (end 145.12 92.59) (width 0.25) (layer "B.Cu") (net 39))
 (segment (start 144.52 96.175292) (end 144.52 93.19) (width 0.25) (layer "B.Cu") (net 39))
 (segment (start 144.5 98.475) (end 144.5 96.79101) (width 0.25) (layer "B.Cu") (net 41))
 (segment (start 145.135718 82.43) (end 146.28 82.43) (width 0.25) (layer "B.Cu") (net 41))
 (segment (start 143.92 92.59) (end 144.52 91.99) (width 0.25) (layer "B.Cu") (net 41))
 (segment (start 147.02 79.87) (end 145.77 78.62) (width 0.25) (layer "B.Cu") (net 41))
 (segment (start 144.52 83.045718) (end 145.135718 82.43) (width 0.25) (layer "B.Cu") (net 41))
 (segment (start 144.52 91.99) (end 144.52 83.045718) (width 0.25) (layer "B.Cu") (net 41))
 (segment (start 144.5 96.79101) (end 141.97 94.26101) (width 0.25) (layer "B.Cu") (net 41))
 (segment (start 141.97 94.26101) (end 141.97 93.24) (width 0.25) (layer "B.Cu") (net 41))
 (segment (start 141.97 93.24) (end 142.62 92.59) (width 0.25) (layer "B.Cu") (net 41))
 (segment (start 147.02 81.69) (end 147.02 79.87) (width 0.25) (layer "B.Cu") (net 41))
 (segment (start 146.28 82.43) (end 147.02 81.69) (width 0.25) (layer "B.Cu") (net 41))
 (segment (start 142.62 92.59) (end 143.92 92.59) (width 0.25) (layer "B.Cu") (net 41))
 (segment (start 144.25 97.16) (end 147.02 94.39) (width 0.25) (layer "F.Cu") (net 42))
 (segment (start 147.02 94.39) (end 147.02 92.57) (width 0.25) (layer "F.Cu") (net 42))
 (segment (start 147.02 92.57) (end 145.77 91.32) (width 0.25) (layer "F.Cu") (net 42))
 (segment (start 144.25 98.725) (end 144.25 97.16) (width 0.25) (layer "F.Cu") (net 42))
 (segment (start 141.46808 83.557638) (end 142.595718 82.43) (width 0.25) (layer "B.Cu") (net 43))
 (segment (start 144 98.475) (end 144 96.926728) (width 0.25) (layer "B.Cu") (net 43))
 (segment (start 144 96.926728) (end 141.46808 94.394808) (width 0.25) (layer "B.Cu") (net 43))
 (segment (start 144.5 82.43) (end 145.77 81.16) (width 0.25) (layer "B.Cu") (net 43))
 (segment (start 141.46808 94.394808) (end 141.46808 83.557638) (width 0.25) (layer "B.Cu") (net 43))
 (segment (start 142.595718 82.43) (end 144.5 82.43) (width 0.25) (layer "B.Cu") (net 43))
 (segment (start 143.75 98.725) (end 143.75 95.937686) (width 0.25) (layer "F.Cu") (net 44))
 (segment (start 145.77 93.917686) (end 145.77 93.86) (width 0.25) (layer "F.Cu") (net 44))
 (segment (start 143.75 95.937686) (end 145.77 93.917686) (width 0.25) (layer "F.Cu") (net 44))
 (segment (start 141.01856 83.37144) (end 143.23 81.16) (width 0.25) (layer "B.Cu") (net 46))
 (segment (start 143 98.475) (end 143 96.562446) (width 0.25) (layer "B.Cu") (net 46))
 (segment (start 141.01856 94.581005) (end 141.01856 83.37144) (width 0.25) (layer "B.Cu") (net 46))
 (segment (start 143 96.562446) (end 141.01856 94.581005) (width 0.25) (layer "B.Cu") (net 46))
 (segment (start 142.5 98.475) (end 142.5 96.698164) (width 0.25) (layer "B.Cu") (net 48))
 (segment (start 140.56904 94.767202) (end 140.56904 81.28096) (width 0.25) (layer "B.Cu") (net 48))
 (segment (start 142.5 96.698164) (end 140.56904 94.767202) (width 0.25) (layer "B.Cu") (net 48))
 (segment (start 140.56904 81.28096) (end 143.23 78.62) (width 0.25) (layer "B.Cu") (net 48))
 (segment (start 140.11952 94.9534) (end 140.11952 79.19048) (width 0.25) (layer "B.Cu") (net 50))
 (segment (start 140.11952 79.19048) (end 143.23 76.08) (width 0.25) (layer "B.Cu") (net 50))
 (segment (start 141.5 98.475) (end 141.5 96.33388) (width 0.25) (layer "B.Cu") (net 50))
 (segment (start 141.5 96.33388) (end 140.11952 94.9534) (width 0.25) (layer "B.Cu") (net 50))
 (segment (start 139.67 95.139597) (end 139.67 77.1) (width 0.25) (layer "B.Cu") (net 52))
 (segment (start 141 98.475) (end 141 96.469598) (width 0.25) (layer "B.Cu") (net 52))
 (segment (start 141 96.469598) (end 139.67 95.139597) (width 0.25) (layer "B.Cu") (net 52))
 (segment (start 139.67 77.1) (end 143.23 73.54) (width 0.25) (layer "B.Cu") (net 52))
 (segment (start 148.945 82.365) (end 148.945 77.096) (width 0.25) (layer "F.Cu") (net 1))
 (segment (start 142.67 90.04) (end 143.795 90.04) (width 0.25) (layer "F.Cu") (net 1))
 (segment (start 150 73.67) (end 150 70.125) (width 0.25) (layer "F.Cu") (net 1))
 (segment (start 151.231 74.81) (end 151.14 74.81) (width 0.25) (layer "F.Cu") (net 1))
 (segment (start 159.25 98.725) (end 159.25 92.13899) (width 0.25) (layer "F.Cu") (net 1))
 (segment (start 157.256499 90.145489) (end 156.283501 90.145489) (width 0.25) (layer "F.Cu") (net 1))
 (segment (start 141.92 94.615) (end 141.92 90.79) (width 0.25) (layer "F.Cu") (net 1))
 (segment (start 157.75 98.725) (end 157.75 95.440362) (width 0.25) (layer "F.Cu") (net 1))
 (segment (start 155.595489 90.833501) (end 155.595489 92.162511) (width 0.25) (layer "F.Cu") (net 1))
 (segment (start 159.25 92.13899) (end 157.256499 90.145489) (width 0.25) (layer "F.Cu") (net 1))
 (segment (start 151.231 74.81) (end 155.5 74.81) (width 0.25) (layer "F.Cu") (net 1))
 (segment (start 149.9921 90.09) (end 148.945 89.0429) (width 0.25) (layer "F.Cu") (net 1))
 (segment (start 141.92 90.79) (end 142.67 90.04) (width 0.25) (layer "F.Cu") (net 1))
 (segment (start 154.23 93.528) (end 154.23 93.86) (width 0.25) (layer "F.Cu") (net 1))
 (segment (start 155.5 74.81) (end 156.77 73.54) (width 0.25) (layer "F.Cu") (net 1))
 (segment (start 157.344149 95.034511) (end 155.404511 95.034511) (width 0.25) (layer "F.Cu") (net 1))
 (segment (start 157.75 95.440362) (end 157.344149 95.034511) (width 0.25) (layer "F.Cu") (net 1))
 (segment (start 142.25 94.945) (end 141.92 94.615) (width 0.25) (layer "F.Cu") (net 1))
 (segment (start 151.14 74.81) (end 150 73.67) (width 0.25) (layer "F.Cu") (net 1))
 (segment (start 143.795 90.04) (end 144.47 89.365) (width 0.25) (layer "F.Cu") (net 1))
 (segment (start 144.47 89.365) (end 144.47 84.94) (width 0.25) (layer "F.Cu") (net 1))
 (segment (start 155.404511 95.034511) (end 154.23 93.86) (width 0.25) (layer "F.Cu") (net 1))
 (segment (start 155.595489 92.162511) (end 154.23 93.528) (width 0.25) (layer "F.Cu") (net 1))
 (segment (start 142.25 98.725) (end 142.25 94.945) (width 0.25) (layer "F.Cu") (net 1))
 (segment (start 148.945 77.096) (end 151.231 74.81) (width 0.25) (layer "F.Cu") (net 1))
 (segment (start 156.283501 90.145489) (end 155.595489 90.833501) (width 0.25) (layer "F.Cu") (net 1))
 (segment (start 143.23 83.7) (end 144.565 82.365) (width 0.25) (layer "F.Cu") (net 1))
 (segment (start 148.945 89.0429) (end 148.945 82.365) (width 0.25) (layer "F.Cu") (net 1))
 (segment (start 144.565 82.365) (end 148.945 82.365) (width 0.25) (layer "F.Cu") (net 1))
 (segment (start 144.47 84.94) (end 143.23 83.7) (width 0.25) (layer "F.Cu") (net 1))
 (via (at 149.9921 90.09) (size 0.8) (drill 0.4) (layers "F.Cu" "B.Cu") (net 1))
 (segment (start 148 95.833879) (end 148 98.475) (width 0.25) (layer "B.Cu") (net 1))
 (segment (start 148.742591 95.091287) (end 148 95.833879) (width 0.25) (layer "B.Cu") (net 1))
 (segment (start 149.9921 91.937499) (end 148.742591 93.187008) (width 0.25) (layer "B.Cu") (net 1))
 (segment (start 149.9921 90.09) (end 149.9921 91.937499) (width 0.25) (layer "B.Cu") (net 1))
 (segment (start 148.742591 93.187008) (end 148.742591 95.091287) (width 0.25) (layer "B.Cu") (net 1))
 (segment (start 158.75 98.725) (end 158.75 93.3) (width 0.2) (layer "F.Cu") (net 2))
 (segment (start 158.75 93.3) (end 156.77 91.32) (width 0.2) (layer "F.Cu") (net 2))
 (segment (start 158.5 87.97) (end 156.77 86.24) (width 0.25) (layer "B.Cu") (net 3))
 (segment (start 158.5 98.475) (end 158.5 87.97) (width 0.25) (layer "B.Cu") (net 3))
 (segment (start 158.25 95.34) (end 156.77 93.86) (width 0.2) (layer "F.Cu") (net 4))
 (segment (start 158.25 98.725) (end 158.25 95.34) (width 0.2) (layer "F.Cu") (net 4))
 (segment (start 158 90.01) (end 158 98.475) (width 0.25) (layer "B.Cu") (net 5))
 (segment (start 156.77 88.78) (end 158 90.01) (width 0.25) (layer "B.Cu") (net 5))
 (segment (start 149 96.105313) (end 149.641631 95.463682) (width 0.25) (layer "B.Cu") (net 26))
 (segment (start 151.22 86.71) (end 154.23 83.7) (width 0.25) (layer "B.Cu") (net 26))
 (segment (start 149.641631 95.463682) (end 149.641631 93.559404) (width 0.25) (layer "B.Cu") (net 26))
 (segment (start 149.641631 93.559404) (end 151.22 91.981035) (width 0.25) (layer "B.Cu") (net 26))
 (segment (start 149 98.475) (end 149 96.105313) (width 0.25) (layer "B.Cu") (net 26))
 (segment (start 151.22 91.981035) (end 151.22 86.71) (width 0.25) (layer "B.Cu") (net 26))
 (segment (start 150.77048 91.794837) (end 149.192111 93.373206) (width 0.25) (layer "B.Cu") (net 28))
 (segment (start 154.23 81.16) (end 151.104 81.16) (width 0.25) (layer "B.Cu") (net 28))
 (segment (start 149.192111 95.277484) (end 148.5 95.969596) (width 0.25) (layer "B.Cu") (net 28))
 (segment (start 150.77048 81.49352) (end 150.77048 91.794837) (width 0.25) (layer "B.Cu") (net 28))
 (segment (start 151.104 81.16) (end 150.77048 81.49352) (width 0.25) (layer "B.Cu") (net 28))
 (segment (start 148.5 95.969596) (end 148.5 98.475) (width 0.25) (layer "B.Cu") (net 28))
 (segment (start 149.192111 93.373206) (end 149.192111 95.277484) (width 0.25) (layer "B.Cu") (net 28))
 (segment (start 141.395 94.915) (end 141.395 90.615) (width 0.25) (layer "F.Cu") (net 49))
 (segment (start 141.395 90.615) (end 143.23 88.78) (width 0.25) (layer "F.Cu") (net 49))
 (segment (start 141.75 98.725) (end 141.75 95.27) (width 0.25) (layer "F.Cu") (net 49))
 (segment (start 141.75 95.27) (end 141.395 94.915) (width 0.25) (layer "F.Cu") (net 49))
 (segment (start 141.25 95.67) (end 140.87 95.29) (width 0.25) (layer "F.Cu") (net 51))
 (segment (start 141.25 98.725) (end 141.25 95.67) (width 0.25) (layer "F.Cu") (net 51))
 (segment (start 140.87 88.6) (end 143.23 86.24) (width 0.25) (layer "F.Cu") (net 51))
 (segment (start 140.87 95.29) (end 140.87 88.6) (width 0.25) (layer "F.Cu") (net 51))
 (segment (start 147.82 88.29) (end 145.77 86.24) (width 0.25) (layer "F.Cu") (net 37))
 (segment (start 145.75 96.791372) (end 147.82 94.721371) (width 0.25) (layer "F.Cu") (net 37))
 (segment (start 145.75 98.725) (end 145.75 96.791372) (width 0.25) (layer "F.Cu") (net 37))
 (segment (start 147.82 94.721371) (end 147.82 88.29) (width 0.25) (layer "F.Cu") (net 37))
 (segment (start 147.42 90.43) (end 145.77 88.78) (width 0.25) (layer "F.Cu") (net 40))
 (segment (start 144.75 98.725) (end 144.75 97.225686) (width 0.25) (layer "F.Cu") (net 40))
 (segment (start 144.75 97.225686) (end 147.42 94.555686) (width 0.25) (layer "F.Cu") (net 40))
 (segment (start 147.42 94.555686) (end 147.42 90.43) (width 0.25) (layer "F.Cu") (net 40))
 (segment (start 143.25 95.872) (end 144.47 94.652) (width 0.25) (layer "F.Cu") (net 45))
 (segment (start 143.25 98.725) (end 143.25 95.872) (width 0.25) (layer "F.Cu") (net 45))
 (segment (start 144.47 92.56) (end 143.23 91.32) (width 0.25) (layer "F.Cu") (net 45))
 (segment (start 144.47 94.652) (end 144.47 92.56) (width 0.25) (layer "F.Cu") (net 45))
 (segment (start 142.75 98.725) (end 142.75 94.34) (width 0.25) (layer "F.Cu") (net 47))
 (segment (start 142.75 94.34) (end 143.23 93.86) (width 0.25) (layer "F.Cu") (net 47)))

